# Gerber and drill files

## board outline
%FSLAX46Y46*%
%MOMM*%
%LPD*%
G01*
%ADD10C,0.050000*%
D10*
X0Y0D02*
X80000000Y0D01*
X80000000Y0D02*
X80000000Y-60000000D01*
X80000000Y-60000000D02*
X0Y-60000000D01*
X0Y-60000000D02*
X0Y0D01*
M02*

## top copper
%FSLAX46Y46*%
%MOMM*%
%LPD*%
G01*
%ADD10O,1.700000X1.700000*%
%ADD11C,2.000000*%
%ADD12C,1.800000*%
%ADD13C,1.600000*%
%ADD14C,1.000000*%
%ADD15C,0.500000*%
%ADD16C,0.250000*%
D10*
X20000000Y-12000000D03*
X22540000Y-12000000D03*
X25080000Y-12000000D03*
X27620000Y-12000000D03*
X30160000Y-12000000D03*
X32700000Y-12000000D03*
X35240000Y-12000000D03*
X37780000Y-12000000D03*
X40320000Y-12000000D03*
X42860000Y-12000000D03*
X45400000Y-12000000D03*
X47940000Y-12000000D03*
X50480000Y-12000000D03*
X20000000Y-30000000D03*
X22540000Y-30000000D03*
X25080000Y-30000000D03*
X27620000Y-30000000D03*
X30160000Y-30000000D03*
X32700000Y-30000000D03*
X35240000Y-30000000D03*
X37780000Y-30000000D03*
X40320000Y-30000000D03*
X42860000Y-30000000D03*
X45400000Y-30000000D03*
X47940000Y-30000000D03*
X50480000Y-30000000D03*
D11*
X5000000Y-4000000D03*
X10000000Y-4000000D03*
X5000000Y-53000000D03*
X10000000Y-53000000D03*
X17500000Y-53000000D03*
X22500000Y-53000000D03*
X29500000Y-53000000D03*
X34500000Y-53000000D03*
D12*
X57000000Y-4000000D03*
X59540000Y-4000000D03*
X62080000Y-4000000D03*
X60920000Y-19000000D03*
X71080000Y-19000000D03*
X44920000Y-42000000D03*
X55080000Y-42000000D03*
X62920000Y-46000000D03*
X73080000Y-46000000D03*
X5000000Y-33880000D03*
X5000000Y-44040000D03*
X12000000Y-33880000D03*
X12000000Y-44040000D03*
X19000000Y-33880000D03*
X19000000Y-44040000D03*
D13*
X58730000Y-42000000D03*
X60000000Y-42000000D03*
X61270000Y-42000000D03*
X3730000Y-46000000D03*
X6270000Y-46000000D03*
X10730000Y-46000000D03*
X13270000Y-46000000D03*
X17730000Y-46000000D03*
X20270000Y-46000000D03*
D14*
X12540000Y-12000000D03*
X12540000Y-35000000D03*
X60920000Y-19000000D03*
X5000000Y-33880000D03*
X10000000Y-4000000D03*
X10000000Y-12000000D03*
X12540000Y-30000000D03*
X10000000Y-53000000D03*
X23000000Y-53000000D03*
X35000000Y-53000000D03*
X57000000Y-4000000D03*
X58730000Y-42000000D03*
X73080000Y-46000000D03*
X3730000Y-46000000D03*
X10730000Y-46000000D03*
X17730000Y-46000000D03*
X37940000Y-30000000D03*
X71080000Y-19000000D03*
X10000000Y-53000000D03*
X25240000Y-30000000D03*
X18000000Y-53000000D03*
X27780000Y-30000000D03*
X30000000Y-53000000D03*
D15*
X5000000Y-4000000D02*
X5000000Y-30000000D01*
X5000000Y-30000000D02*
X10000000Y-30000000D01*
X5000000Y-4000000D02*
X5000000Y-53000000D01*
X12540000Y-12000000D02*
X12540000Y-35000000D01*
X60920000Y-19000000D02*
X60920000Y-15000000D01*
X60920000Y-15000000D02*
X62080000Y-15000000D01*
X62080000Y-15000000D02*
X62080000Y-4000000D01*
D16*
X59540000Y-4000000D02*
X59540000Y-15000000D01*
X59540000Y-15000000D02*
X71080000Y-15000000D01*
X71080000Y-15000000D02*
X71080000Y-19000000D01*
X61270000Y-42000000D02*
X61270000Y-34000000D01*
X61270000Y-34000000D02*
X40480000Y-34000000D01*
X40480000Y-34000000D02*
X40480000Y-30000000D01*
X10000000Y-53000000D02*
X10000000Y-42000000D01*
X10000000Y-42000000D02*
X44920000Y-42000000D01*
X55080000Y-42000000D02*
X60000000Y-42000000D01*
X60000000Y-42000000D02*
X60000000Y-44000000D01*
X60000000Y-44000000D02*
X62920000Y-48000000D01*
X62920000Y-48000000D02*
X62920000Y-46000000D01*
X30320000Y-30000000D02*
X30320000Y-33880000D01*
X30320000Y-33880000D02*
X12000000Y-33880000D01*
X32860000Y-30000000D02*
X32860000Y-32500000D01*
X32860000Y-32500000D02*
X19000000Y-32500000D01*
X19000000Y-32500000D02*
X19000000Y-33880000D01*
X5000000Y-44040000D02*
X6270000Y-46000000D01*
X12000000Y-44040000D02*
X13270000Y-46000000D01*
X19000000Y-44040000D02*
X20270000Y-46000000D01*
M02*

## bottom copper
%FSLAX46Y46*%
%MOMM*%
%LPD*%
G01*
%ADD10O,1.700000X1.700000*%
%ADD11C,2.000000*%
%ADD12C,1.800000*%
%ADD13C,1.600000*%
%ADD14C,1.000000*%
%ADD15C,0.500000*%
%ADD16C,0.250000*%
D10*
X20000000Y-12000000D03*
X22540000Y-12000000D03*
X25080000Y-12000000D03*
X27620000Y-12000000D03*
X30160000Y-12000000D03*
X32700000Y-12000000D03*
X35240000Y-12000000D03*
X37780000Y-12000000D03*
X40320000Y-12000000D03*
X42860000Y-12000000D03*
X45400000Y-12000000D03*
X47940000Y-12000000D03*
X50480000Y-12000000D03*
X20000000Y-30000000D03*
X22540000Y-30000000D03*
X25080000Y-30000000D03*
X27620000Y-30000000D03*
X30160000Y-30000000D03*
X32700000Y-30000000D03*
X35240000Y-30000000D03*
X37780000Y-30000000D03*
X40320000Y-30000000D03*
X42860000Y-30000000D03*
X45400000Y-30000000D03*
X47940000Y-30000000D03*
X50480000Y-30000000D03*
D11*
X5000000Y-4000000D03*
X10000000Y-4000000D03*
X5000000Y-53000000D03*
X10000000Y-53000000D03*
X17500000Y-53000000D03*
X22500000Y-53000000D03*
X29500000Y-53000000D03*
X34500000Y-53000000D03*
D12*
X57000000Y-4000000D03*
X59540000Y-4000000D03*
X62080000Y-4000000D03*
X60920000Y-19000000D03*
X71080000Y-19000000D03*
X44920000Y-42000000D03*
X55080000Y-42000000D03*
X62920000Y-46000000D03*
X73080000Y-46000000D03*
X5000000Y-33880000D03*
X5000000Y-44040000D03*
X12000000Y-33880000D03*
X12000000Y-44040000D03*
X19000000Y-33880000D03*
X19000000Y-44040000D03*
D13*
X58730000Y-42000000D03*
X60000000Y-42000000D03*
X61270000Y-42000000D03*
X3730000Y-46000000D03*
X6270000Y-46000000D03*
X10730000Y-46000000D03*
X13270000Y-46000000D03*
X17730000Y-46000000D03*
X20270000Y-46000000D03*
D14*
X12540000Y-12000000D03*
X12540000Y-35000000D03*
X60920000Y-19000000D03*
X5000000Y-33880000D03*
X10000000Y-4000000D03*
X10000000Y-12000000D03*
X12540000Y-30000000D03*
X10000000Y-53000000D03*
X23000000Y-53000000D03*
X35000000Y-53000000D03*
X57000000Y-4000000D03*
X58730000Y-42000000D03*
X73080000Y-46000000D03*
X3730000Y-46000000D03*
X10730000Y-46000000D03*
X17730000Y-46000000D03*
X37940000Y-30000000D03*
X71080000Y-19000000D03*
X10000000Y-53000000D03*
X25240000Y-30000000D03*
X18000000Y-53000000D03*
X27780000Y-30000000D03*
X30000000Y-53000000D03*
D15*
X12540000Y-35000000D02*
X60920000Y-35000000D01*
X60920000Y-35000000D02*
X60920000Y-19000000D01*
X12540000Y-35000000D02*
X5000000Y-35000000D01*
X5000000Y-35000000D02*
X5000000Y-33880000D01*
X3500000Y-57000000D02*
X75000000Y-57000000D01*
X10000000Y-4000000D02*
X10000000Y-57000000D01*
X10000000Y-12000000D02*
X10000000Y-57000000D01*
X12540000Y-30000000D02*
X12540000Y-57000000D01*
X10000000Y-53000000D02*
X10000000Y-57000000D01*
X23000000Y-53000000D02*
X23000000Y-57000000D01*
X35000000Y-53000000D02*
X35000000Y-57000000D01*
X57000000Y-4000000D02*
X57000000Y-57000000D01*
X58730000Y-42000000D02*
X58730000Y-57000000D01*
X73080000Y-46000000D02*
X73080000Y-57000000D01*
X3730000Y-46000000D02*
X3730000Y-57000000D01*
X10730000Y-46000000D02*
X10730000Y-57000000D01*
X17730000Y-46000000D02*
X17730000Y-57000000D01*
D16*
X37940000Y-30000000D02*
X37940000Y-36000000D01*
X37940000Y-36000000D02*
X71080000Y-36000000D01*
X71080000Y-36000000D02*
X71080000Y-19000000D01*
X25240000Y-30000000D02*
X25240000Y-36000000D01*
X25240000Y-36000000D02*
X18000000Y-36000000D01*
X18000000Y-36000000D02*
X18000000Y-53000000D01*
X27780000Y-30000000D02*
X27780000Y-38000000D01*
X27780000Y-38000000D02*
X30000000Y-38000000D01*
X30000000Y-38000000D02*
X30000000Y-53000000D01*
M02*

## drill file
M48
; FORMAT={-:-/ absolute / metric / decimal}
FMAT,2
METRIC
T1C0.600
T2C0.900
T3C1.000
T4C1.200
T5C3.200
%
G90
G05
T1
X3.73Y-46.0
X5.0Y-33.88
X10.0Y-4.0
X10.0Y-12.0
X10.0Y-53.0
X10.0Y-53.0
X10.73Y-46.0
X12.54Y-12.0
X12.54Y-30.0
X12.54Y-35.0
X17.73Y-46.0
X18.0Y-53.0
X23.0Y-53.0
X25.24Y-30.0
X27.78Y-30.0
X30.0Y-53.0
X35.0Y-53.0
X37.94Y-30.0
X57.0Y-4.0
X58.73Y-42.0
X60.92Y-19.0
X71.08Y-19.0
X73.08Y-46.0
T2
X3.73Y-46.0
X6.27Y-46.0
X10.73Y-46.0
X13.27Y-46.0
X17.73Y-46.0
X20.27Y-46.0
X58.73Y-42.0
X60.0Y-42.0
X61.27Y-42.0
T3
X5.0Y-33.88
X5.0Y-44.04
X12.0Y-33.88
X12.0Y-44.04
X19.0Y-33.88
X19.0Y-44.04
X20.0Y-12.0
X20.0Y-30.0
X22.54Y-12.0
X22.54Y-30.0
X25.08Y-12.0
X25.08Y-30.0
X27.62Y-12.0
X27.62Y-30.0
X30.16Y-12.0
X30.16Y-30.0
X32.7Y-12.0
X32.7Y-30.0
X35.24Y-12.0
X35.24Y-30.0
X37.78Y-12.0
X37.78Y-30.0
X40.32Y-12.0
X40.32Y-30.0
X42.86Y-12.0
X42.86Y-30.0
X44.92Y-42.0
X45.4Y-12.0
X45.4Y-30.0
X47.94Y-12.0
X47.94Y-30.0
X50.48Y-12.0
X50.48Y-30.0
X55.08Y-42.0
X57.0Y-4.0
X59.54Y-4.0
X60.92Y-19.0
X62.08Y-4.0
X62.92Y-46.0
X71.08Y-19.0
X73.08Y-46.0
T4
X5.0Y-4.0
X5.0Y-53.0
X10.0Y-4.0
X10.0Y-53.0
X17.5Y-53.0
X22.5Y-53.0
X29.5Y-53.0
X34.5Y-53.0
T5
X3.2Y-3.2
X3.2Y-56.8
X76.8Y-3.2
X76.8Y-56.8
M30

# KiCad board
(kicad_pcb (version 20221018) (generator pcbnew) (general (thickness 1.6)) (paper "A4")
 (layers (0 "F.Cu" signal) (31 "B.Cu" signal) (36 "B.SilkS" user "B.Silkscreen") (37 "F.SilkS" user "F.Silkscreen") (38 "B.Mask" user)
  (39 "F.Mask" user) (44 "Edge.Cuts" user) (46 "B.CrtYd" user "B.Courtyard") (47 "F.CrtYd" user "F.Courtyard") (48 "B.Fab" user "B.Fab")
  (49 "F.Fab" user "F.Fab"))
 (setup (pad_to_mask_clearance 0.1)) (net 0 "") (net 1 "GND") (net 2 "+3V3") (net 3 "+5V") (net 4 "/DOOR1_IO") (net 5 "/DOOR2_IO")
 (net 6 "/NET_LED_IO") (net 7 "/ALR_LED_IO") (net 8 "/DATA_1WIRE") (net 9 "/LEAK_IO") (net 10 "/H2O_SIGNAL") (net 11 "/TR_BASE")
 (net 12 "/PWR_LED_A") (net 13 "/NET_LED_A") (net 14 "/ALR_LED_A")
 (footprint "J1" (layer "F.Cu") (at 25.240 12.000)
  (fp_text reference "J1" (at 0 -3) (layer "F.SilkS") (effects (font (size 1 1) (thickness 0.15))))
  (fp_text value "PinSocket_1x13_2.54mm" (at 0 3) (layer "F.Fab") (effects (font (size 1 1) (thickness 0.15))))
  (pad "1" thru_hole oval (at -5.240 0.000) (size 1.7 1.7) (drill 1.0) (layers "F.Cu" "B.Cu" "F.Mask" "B.Mask") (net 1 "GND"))
  (pad "2" thru_hole oval (at -2.700 0.000) (size 1.7 1.7) (drill 1.0) (layers "F.Cu" "B.Cu" "F.Mask" "B.Mask") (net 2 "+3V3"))
  (pad "3" thru_hole oval (at -0.160 0.000) (size 1.7 1.7) (drill 1.0) (layers "F.Cu" "B.Cu" "F.Mask" "B.Mask"))
  (pad "4" thru_hole oval (at 2.380 0.000) (size 1.7 1.7) (drill 1.0) (layers "F.Cu" "B.Cu" "F.Mask" "B.Mask"))
  (pad "5" thru_hole oval (at 4.920 0.000) (size 1.7 1.7) (drill 1.0) (layers "F.Cu" "B.Cu" "F.Mask" "B.Mask"))
  (pad "6" thru_hole oval (at 7.460 0.000) (size 1.7 1.7) (drill 1.0) (layers "F.Cu" "B.Cu" "F.Mask" "B.Mask"))
  (pad "7" thru_hole oval (at 10.000 0.000) (size 1.7 1.7) (drill 1.0) (layers "F.Cu" "B.Cu" "F.Mask" "B.Mask"))
  (pad "8" thru_hole oval (at 12.540 0.000) (size 1.7 1.7) (drill 1.0) (layers "F.Cu" "B.Cu" "F.Mask" "B.Mask"))
  (pad "9" thru_hole oval (at 15.080 0.000) (size 1.7 1.7) (drill 1.0) (layers "F.Cu" "B.Cu" "F.Mask" "B.Mask"))
  (pad "10" thru_hole oval (at 17.620 0.000) (size 1.7 1.7) (drill 1.0) (layers "F.Cu" "B.Cu" "F.Mask" "B.Mask"))
  (pad "11" thru_hole oval (at 20.160 0.000) (size 1.7 1.7) (drill 1.0) (layers "F.Cu" "B.Cu" "F.Mask" "B.Mask"))
  (pad "12" thru_hole oval (at 22.700 0.000) (size 1.7 1.7) (drill 1.0) (layers "F.Cu" "B.Cu" "F.Mask" "B.Mask"))
  (pad "13" thru_hole oval (at 25.240 0.000) (size 1.7 1.7) (drill 1.0) (layers "F.Cu" "B.Cu" "F.Mask" "B.Mask")))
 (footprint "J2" (layer "F.Cu") (at 25.240 30.000)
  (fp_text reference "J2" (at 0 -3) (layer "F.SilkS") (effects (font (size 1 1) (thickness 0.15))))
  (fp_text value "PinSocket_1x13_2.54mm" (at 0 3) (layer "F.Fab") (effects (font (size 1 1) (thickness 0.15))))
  (pad "1" thru_hole oval (at -5.240 0.000) (size 1.7 1.7) (drill 1.0) (layers "F.Cu" "B.Cu" "F.Mask" "B.Mask") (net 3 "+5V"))
  (pad "2" thru_hole oval (at -2.700 0.000) (size 1.7 1.7) (drill 1.0) (layers "F.Cu" "B.Cu" "F.Mask" "B.Mask") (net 1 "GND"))
  (pad "3" thru_hole oval (at -0.160 0.000) (size 1.7 1.7) (drill 1.0) (layers "F.Cu" "B.Cu" "F.Mask" "B.Mask"))
  (pad "4" thru_hole oval (at 2.380 0.000) (size 1.7 1.7) (drill 1.0) (layers "F.Cu" "B.Cu" "F.Mask" "B.Mask"))
  (pad "5" thru_hole oval (at 4.920 0.000) (size 1.7 1.7) (drill 1.0) (layers "F.Cu" "B.Cu" "F.Mask" "B.Mask"))
  (pad "6" thru_hole oval (at 7.460 0.000) (size 1.7 1.7) (drill 1.0) (layers "F.Cu" "B.Cu" "F.Mask" "B.Mask"))
  (pad "7" thru_hole oval (at 10.000 0.000) (size 1.7 1.7) (drill 1.0) (layers "F.Cu" "B.Cu" "F.Mask" "B.Mask") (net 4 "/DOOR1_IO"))
  (pad "8" thru_hole oval (at 12.540 0.000) (size 1.7 1.7) (drill 1.0) (layers "F.Cu" "B.Cu" "F.Mask" "B.Mask") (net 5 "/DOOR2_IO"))
  (pad "9" thru_hole oval (at 15.080 0.000) (size 1.7 1.7) (drill 1.0) (layers "F.Cu" "B.Cu" "F.Mask" "B.Mask") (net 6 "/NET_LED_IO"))
  (pad "10" thru_hole oval (at 17.620 0.000) (size 1.7 1.7) (drill 1.0) (layers "F.Cu" "B.Cu" "F.Mask" "B.Mask") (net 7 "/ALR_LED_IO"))
  (pad "11" thru_hole oval (at 20.160 0.000) (size 1.7 1.7) (drill 1.0) (layers "F.Cu" "B.Cu" "F.Mask" "B.Mask"))
  (pad "12" thru_hole oval (at 22.700 0.000) (size 1.7 1.7) (drill 1.0) (layers "F.Cu" "B.Cu" "F.Mask" "B.Mask") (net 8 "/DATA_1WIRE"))
  (pad "13" thru_hole oval (at 25.240 0.000) (size 1.7 1.7) (drill 1.0) (layers "F.Cu" "B.Cu" "F.Mask" "B.Mask") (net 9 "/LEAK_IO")))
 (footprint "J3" (layer "F.Cu") (at 7.500 4.000)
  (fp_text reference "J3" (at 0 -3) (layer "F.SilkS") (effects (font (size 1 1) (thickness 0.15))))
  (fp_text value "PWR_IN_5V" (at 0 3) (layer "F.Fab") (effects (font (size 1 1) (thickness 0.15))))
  (pad "1" thru_hole circle (at -2.500 0.000) (size 2.0 2.0) (drill 1.2) (layers "F.Cu" "B.Cu" "F.Mask" "B.Mask") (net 3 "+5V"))
  (pad "2" thru_hole circle (at 2.500 0.000) (size 2.0 2.0) (drill 1.2) (layers "F.Cu" "B.Cu" "F.Mask" "B.Mask") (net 1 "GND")))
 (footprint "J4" (layer "F.Cu") (at 7.500 53.000)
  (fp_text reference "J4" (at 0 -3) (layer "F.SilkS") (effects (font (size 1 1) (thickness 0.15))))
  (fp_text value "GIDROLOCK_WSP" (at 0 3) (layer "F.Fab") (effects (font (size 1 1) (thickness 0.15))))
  (pad "1" thru_hole circle (at -2.500 0.000) (size 2.0 2.0) (drill 1.2) (layers "F.Cu" "B.Cu" "F.Mask" "B.Mask") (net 3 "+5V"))
  (pad "2" thru_hole circle (at 2.500 0.000) (size 2.0 2.0) (drill 1.2) (layers "F.Cu" "B.Cu" "F.Mask" "B.Mask") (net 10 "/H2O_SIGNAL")))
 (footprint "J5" (layer "F.Cu") (at 20.000 53.000)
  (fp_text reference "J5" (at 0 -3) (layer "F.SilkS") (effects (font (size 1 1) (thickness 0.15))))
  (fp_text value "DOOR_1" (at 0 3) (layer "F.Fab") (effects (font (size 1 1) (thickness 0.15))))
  (pad "1" thru_hole circle (at -2.500 0.000) (size 2.0 2.0) (drill 1.2) (layers "F.Cu" "B.Cu" "F.Mask" "B.Mask") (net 4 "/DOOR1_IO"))
  (pad "2" thru_hole circle (at 2.500 0.000) (size 2.0 2.0) (drill 1.2) (layers "F.Cu" "B.Cu" "F.Mask" "B.Mask") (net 1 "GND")))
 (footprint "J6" (layer "F.Cu") (at 32.000 53.000)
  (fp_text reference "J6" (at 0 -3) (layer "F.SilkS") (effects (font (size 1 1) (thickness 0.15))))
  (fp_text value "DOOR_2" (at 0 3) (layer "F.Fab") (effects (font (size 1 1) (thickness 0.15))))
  (pad "1" thru_hole circle (at -2.500 0.000) (size 2.0 2.0) (drill 1.2) (layers "F.Cu" "B.Cu" "F.Mask" "B.Mask") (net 5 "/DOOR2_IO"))
  (pad "2" thru_hole circle (at 2.500 0.000) (size 2.0 2.0) (drill 1.2) (layers "F.Cu" "B.Cu" "F.Mask" "B.Mask") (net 1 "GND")))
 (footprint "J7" (layer "F.Cu") (at 59.540 4.000)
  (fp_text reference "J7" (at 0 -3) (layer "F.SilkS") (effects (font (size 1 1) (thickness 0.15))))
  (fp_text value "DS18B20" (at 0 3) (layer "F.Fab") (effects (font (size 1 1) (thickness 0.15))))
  (pad "1" thru_hole circle (at -2.540 0.000) (size 1.8 1.8) (drill 1.0) (layers "F.Cu" "B.Cu" "F.Mask" "B.Mask") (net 1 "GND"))
  (pad "2" thru_hole circle (at 0.000 0.000) (size 1.8 1.8) (drill 1.0) (layers "F.Cu" "B.Cu" "F.Mask" "B.Mask") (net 8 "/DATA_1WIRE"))
  (pad "3" thru_hole circle (at 2.540 0.000) (size 1.8 1.8) (drill 1.0) (layers "F.Cu" "B.Cu" "F.Mask" "B.Mask") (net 2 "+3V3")))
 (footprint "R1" (layer "F.Cu") (at 66.000 19.000)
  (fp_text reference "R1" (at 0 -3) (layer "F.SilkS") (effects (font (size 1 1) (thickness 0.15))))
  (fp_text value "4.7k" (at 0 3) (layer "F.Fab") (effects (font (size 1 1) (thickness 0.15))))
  (pad "1" thru_hole circle (at -5.080 0.000) (size 1.8 1.8) (drill 1.0) (layers "F.Cu" "B.Cu" "F.Mask" "B.Mask") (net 2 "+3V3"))
  (pad "2" thru_hole circle (at 5.080 0.000) (size 1.8 1.8) (drill 1.0) (layers "F.Cu" "B.Cu" "F.Mask" "B.Mask") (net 8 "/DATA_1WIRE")))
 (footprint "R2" (layer "F.Cu") (at 50.000 42.000)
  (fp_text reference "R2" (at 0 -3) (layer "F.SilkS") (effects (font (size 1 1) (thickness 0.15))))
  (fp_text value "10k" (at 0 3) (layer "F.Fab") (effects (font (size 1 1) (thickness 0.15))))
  (pad "1" thru_hole circle (at -5.080 0.000) (size 1.8 1.8) (drill 1.0) (layers "F.Cu" "B.Cu" "F.Mask" "B.Mask") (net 10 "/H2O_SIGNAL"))
  (pad "2" thru_hole circle (at 5.080 0.000) (size 1.8 1.8) (drill 1.0) (layers "F.Cu" "B.Cu" "F.Mask" "B.Mask") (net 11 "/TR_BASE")))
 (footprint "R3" (layer "F.Cu") (at 68.000 46.000)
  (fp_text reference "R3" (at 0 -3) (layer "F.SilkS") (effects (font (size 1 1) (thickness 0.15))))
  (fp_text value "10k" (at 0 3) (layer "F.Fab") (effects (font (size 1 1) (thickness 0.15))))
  (pad "1" thru_hole circle (at -5.080 0.000) (size 1.8 1.8) (drill 1.0) (layers "F.Cu" "B.Cu" "F.Mask" "B.Mask") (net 11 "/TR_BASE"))
  (pad "2" thru_hole circle (at 5.080 0.000) (size 1.8 1.8) (drill 1.0) (layers "F.Cu" "B.Cu" "F.Mask" "B.Mask") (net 1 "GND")))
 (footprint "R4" (layer "F.Cu") (at 5.000 38.960)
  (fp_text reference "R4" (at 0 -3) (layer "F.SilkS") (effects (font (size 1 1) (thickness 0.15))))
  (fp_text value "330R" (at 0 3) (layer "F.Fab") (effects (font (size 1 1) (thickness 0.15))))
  (pad "1" thru_hole circle (at 0.000 -5.080) (size 1.8 1.8) (drill 1.0) (layers "F.Cu" "B.Cu" "F.Mask" "B.Mask") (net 2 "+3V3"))
  (pad "2" thru_hole circle (at 0.000 5.080) (size 1.8 1.8) (drill 1.0) (layers "F.Cu" "B.Cu" "F.Mask" "B.Mask") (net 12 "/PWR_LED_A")))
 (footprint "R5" (layer "F.Cu") (at 12.000 38.960)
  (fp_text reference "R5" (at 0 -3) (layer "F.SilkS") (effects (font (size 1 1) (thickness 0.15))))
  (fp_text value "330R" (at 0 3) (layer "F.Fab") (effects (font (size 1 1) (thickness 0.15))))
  (pad "1" thru_hole circle (at 0.000 -5.080) (size 1.8 1.8) (drill 1.0) (layers "F.Cu" "B.Cu" "F.Mask" "B.Mask") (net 6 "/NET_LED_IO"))
  (pad "2" thru_hole circle (at 0.000 5.080) (size 1.8 1.8) (drill 1.0) (layers "F.Cu" "B.Cu" "F.Mask" "B.Mask") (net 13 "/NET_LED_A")))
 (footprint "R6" (layer "F.Cu") (at 19.000 38.960)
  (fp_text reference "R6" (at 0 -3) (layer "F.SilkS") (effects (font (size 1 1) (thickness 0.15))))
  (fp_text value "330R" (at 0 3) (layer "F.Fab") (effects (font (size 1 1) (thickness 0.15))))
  (pad "1" thru_hole circle (at 0.000 -5.080) (size 1.8 1.8) (drill 1.0) (layers "F.Cu" "B.Cu" "F.Mask" "B.Mask") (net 7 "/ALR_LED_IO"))
  (pad "2" thru_hole circle (at 0.000 5.080) (size 1.8 1.8) (drill 1.0) (layers "F.Cu" "B.Cu" "F.Mask" "B.Mask") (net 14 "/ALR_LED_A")))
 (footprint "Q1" (layer "F.Cu") (at 60.000 42.000)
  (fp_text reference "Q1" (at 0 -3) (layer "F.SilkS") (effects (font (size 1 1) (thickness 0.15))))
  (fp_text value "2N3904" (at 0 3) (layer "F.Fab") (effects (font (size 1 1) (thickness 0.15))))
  (pad "1" thru_hole circle (at -1.270 0.000) (size 1.6 1.6) (drill 0.9) (layers "F.Cu" "B.Cu" "F.Mask" "B.Mask") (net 1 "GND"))
  (pad "2" thru_hole circle (at 0.000 0.000) (size 1.6 1.6) (drill 0.9) (layers "F.Cu" "B.Cu" "F.Mask" "B.Mask") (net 11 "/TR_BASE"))
  (pad "3" thru_hole circle (at 1.270 0.000) (size 1.6 1.6) (drill 0.9) (layers "F.Cu" "B.Cu" "F.Mask" "B.Mask") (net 9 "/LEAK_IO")))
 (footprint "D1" (layer "F.Cu") (at 5.000 46.000)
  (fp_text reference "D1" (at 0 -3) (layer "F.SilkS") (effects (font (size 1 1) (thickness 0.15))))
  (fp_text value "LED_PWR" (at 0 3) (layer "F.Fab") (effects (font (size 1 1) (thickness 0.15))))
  (pad "K" thru_hole circle (at -1.270 0.000) (size 1.6 1.6) (drill 0.9) (layers "F.Cu" "B.Cu" "F.Mask" "B.Mask") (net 1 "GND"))
  (pad "A" thru_hole circle (at 1.270 0.000) (size 1.6 1.6) (drill 0.9) (layers "F.Cu" "B.Cu" "F.Mask" "B.Mask") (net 12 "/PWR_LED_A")))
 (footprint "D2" (layer "F.Cu") (at 12.000 46.000)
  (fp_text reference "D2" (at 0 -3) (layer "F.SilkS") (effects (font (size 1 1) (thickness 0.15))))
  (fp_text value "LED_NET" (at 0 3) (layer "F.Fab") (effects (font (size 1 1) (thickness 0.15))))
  (pad "K" thru_hole circle (at -1.270 0.000) (size 1.6 1.6) (drill 0.9) (layers "F.Cu" "B.Cu" "F.Mask" "B.Mask") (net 1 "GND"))
  (pad "A" thru_hole circle (at 1.270 0.000) (size 1.6 1.6) (drill 0.9) (layers "F.Cu" "B.Cu" "F.Mask" "B.Mask") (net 13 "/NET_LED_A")))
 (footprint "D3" (layer "F.Cu") (at 19.000 46.000)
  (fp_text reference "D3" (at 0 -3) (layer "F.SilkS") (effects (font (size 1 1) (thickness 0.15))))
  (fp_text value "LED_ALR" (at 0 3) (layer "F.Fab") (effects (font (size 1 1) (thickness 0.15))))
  (pad "K" thru_hole circle (at -1.270 0.000) (size 1.6 1.6) (drill 0.9) (layers "F.Cu" "B.Cu" "F.Mask" "B.Mask") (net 1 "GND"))
  (pad "A" thru_hole circle (at 1.270 0.000) (size 1.6 1.6) (drill 0.9) (layers "F.Cu" "B.Cu" "F.Mask" "B.Mask") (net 14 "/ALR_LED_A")))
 (segment (start 5.000 4.000) (end 5.000 30.000) (width 0.50) (layer "F.Cu") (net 3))
 (segment (start 5.000 30.000) (end 10.000 30.000) (width 0.50) (layer "F.Cu") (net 3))
 (segment (start 5.000 4.000) (end 5.000 53.000) (width 0.50) (layer "F.Cu") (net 3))
 (via (at 12.540 12.000) (size 1.0) (drill 0.6) (layers "F.Cu" "B.Cu") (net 2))
 (segment (start 12.540 12.000) (end 12.540 35.000) (width 0.50) (layer "F.Cu") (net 2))
 (via (at 12.540 35.000) (size 1.0) (drill 0.6) (layers "F.Cu" "B.Cu") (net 2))
 (segment (start 12.540 35.000) (end 60.920 35.000) (width 0.50) (layer "B.Cu") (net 2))
 (segment (start 60.920 35.000) (end 60.920 19.000) (width 0.50) (layer "B.Cu") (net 2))
 (via (at 60.920 19.000) (size 1.0) (drill 0.6) (layers "F.Cu" "B.Cu") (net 2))
 (segment (start 60.920 19.000) (end 60.920 15.000) (width 0.50) (layer "F.Cu") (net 2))
 (segment (start 60.920 15.000) (end 62.080 15.000) (width 0.50) (layer "F.Cu") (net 2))
 (segment (start 62.080 15.000) (end 62.080 4.000) (width 0.50) (layer "F.Cu") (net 2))
 (segment (start 12.540 35.000) (end 5.000 35.000) (width 0.50) (layer "B.Cu") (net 2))
 (segment (start 5.000 35.000) (end 5.000 33.880) (width 0.50) (layer "B.Cu") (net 2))
 (via (at 5.000 33.880) (size 1.0) (drill 0.6) (layers "F.Cu" "B.Cu") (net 2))
 (via (at 10.000 4.000) (size 1.0) (drill 0.6) (layers "F.Cu" "B.Cu") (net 1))
 (via (at 10.000 12.000) (size 1.0) (drill 0.6) (layers "F.Cu" "B.Cu") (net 1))
 (via (at 12.540 30.000) (size 1.0) (drill 0.6) (layers "F.Cu" "B.Cu") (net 1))
 (via (at 10.000 53.000) (size 1.0) (drill 0.6) (layers "F.Cu" "B.Cu") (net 1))
 (via (at 23.000 53.000) (size 1.0) (drill 0.6) (layers "F.Cu" "B.Cu") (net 1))
 (via (at 35.000 53.000) (size 1.0) (drill 0.6) (layers "F.Cu" "B.Cu") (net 1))
 (via (at 57.000 4.000) (size 1.0) (drill 0.6) (layers "F.Cu" "B.Cu") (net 1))
 (via (at 58.730 42.000) (size 1.0) (drill 0.6) (layers "F.Cu" "B.Cu") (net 1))
 (via (at 73.080 46.000) (size 1.0) (drill 0.6) (layers "F.Cu" "B.Cu") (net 1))
 (via (at 3.730 46.000) (size 1.0) (drill 0.6) (layers "F.Cu" "B.Cu") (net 1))
 (via (at 10.730 46.000) (size 1.0) (drill 0.6) (layers "F.Cu" "B.Cu") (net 1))
 (via (at 17.730 46.000) (size 1.0) (drill 0.6) (layers "F.Cu" "B.Cu") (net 1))
 (segment (start 3.500 57.000) (end 75.000 57.000) (width 0.50) (layer "B.Cu") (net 1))
 (segment (start 10.000 4.000) (end 10.000 57.000) (width 0.50) (layer "B.Cu") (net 1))
 (segment (start 10.000 12.000) (end 10.000 57.000) (width 0.50) (layer "B.Cu") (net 1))
 (segment (start 12.540 30.000) (end 12.540 57.000) (width 0.50) (layer "B.Cu") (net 1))
 (segment (start 10.000 53.000) (end 10.000 57.000) (width 0.50) (layer "B.Cu") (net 1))
 (segment (start 23.000 53.000) (end 23.000 57.000) (width 0.50) (layer "B.Cu") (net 1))
 (segment (start 35.000 53.000) (end 35.000 57.000) (width 0.50) (layer "B.Cu") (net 1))
 (segment (start 57.000 4.000) (end 57.000 57.000) (width 0.50) (layer "B.Cu") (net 1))
 (segment (start 58.730 42.000) (end 58.730 57.000) (width 0.50) (layer "B.Cu") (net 1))
 (segment (start 73.080 46.000) (end 73.080 57.000) (width 0.50) (layer "B.Cu") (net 1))
 (segment (start 3.730 46.000) (end 3.730 57.000) (width 0.50) (layer "B.Cu") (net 1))
 (segment (start 10.730 46.000) (end 10.730 57.000) (width 0.50) (layer "B.Cu") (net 1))
 (segment (start 17.730 46.000) (end 17.730 57.000) (width 0.50) (layer "B.Cu") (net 1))
 (via (at 37.940 30.000) (size 1.0) (drill 0.6) (layers "F.Cu" "B.Cu") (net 8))
 (segment (start 37.940 30.000) (end 37.940 36.000) (width 0.25) (layer "B.Cu") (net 8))
 (segment (start 37.940 36.000) (end 71.080 36.000) (width 0.25) (layer "B.Cu") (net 8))
 (segment (start 71.080 36.000) (end 71.080 19.000) (width 0.25) (layer "B.Cu") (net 8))
 (via (at 71.080 19.000) (size 1.0) (drill 0.6) (layers "F.Cu" "B.Cu") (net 8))
 (segment (start 59.540 4.000) (end 59.540 15.000) (width 0.25) (layer "F.Cu") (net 8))
 (segment (start 59.540 15.000) (end 71.080 15.000) (width 0.25) (layer "F.Cu") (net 8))
 (segment (start 71.080 15.000) (end 71.080 19.000) (width 0.25) (layer "F.Cu") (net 8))
 (segment (start 61.270 42.000) (end 61.270 34.000) (width 0.25) (layer "F.Cu") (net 9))
 (segment (start 61.270 34.000) (end 40.480 34.000) (width 0.25) (layer "F.Cu") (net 9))
 (segment (start 40.480 34.000) (end 40.480 30.000) (width 0.25) (layer "F.Cu") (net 9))
 (via (at 10.000 53.000) (size 1.0) (drill 0.6) (layers "F.Cu" "B.Cu") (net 10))
 (segment (start 10.000 53.000) (end 10.000 42.000) (width 0.25) (layer "F.Cu") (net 10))
 (segment (start 10.000 42.000) (end 44.920 42.000) (width 0.25) (layer "F.Cu") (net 10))
 (segment (start 55.080 42.000) (end 60.000 42.000) (width 0.25) (layer "F.Cu") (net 11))
 (segment (start 60.000 42.000) (end 60.000 44.000) (width 0.25) (layer "F.Cu") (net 11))
 (segment (start 60.000 44.000) (end 62.920 48.000) (width 0.25) (layer "F.Cu") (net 11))
 (segment (start 62.920 48.000) (end 62.920 46.000) (width 0.25) (layer "F.Cu") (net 11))
 (via (at 25.240 30.000) (size 1.0) (drill 0.6) (layers "F.Cu" "B.Cu") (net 4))
 (segment (start 25.240 30.000) (end 25.240 36.000) (width 0.25) (layer "B.Cu") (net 4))
 (segment (start 25.240 36.000) (end 18.000 36.000) (width 0.25) (layer "B.Cu") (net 4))
 (segment (start 18.000 36.000) (end 18.000 53.000) (width 0.25) (layer "B.Cu") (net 4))
 (via (at 18.000 53.000) (size 1.0) (drill 0.6) (layers "F.Cu" "B.Cu") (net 4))
 (via (at 27.780 30.000) (size 1.0) (drill 0.6) (layers "F.Cu" "B.Cu") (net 5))
 (segment (start 27.780 30.000) (end 27.780 38.000) (width 0.25) (layer "B.Cu") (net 5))
 (segment (start 27.780 38.000) (end 30.000 38.000) (width 0.25) (layer "B.Cu") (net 5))
 (segment (start 30.000 38.000) (end 30.000 53.000) (width 0.25) (layer "B.Cu") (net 5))
 (via (at 30.000 53.000) (size 1.0) (drill 0.6) (layers "F.Cu" "B.Cu") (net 5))
 (segment (start 30.320 30.000) (end 30.320 33.880) (width 0.25) (layer "F.Cu") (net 6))
 (segment (start 30.320 33.880) (end 12.000 33.880) (width 0.25) (layer "F.Cu") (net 6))
 (segment (start 32.860 30.000) (end 32.860 32.500) (width 0.25) (layer "F.Cu") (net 7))
 (segment (start 32.860 32.500) (end 19.000 32.500) (width 0.25) (layer "F.Cu") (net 7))
 (segment (start 19.000 32.500) (end 19.000 33.880) (width 0.25) (layer "F.Cu") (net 7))
 (segment (start 5.000 44.040) (end 6.270 46.000) (width 0.25) (layer "F.Cu") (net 12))
 (segment (start 12.000 44.040) (end 13.270 46.000) (width 0.25) (layer "F.Cu") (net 13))
 (segment (start 19.000 44.040) (end 20.270 46.000) (width 0.25) (layer "F.Cu") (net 14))
 (gr_line (start 0 0) (end 80.0 0) (layer "Edge.Cuts") (width 0.05))
 (gr_line (start 80.0 0) (end 80.0 60.0) (layer "Edge.Cuts") (width 0.05))
 (gr_line (start 80.0 60.0) (end 0 60.0) (layer "Edge.Cuts") (width 0.05))
 (gr_line (start 0 60.0) (end 0 0) (layer "Edge.Cuts") (width 0.05))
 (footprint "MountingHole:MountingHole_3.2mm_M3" (layer "F.Cu") (at 3.2 3.2)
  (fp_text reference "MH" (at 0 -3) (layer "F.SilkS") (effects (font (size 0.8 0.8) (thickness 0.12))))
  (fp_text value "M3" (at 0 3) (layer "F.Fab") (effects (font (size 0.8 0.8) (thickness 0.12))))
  (pad "" np_thru_hole circle (at 0 0) (size 3.2 3.2) (drill 3.2) (layers "*.Cu" "*.Mask")))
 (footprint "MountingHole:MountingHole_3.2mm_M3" (layer "F.Cu") (at 76.8 3.2)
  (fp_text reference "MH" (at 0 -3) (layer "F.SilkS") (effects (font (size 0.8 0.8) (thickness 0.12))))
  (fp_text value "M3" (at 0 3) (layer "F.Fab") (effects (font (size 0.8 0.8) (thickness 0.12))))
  (pad "" np_thru_hole circle (at 0 0) (size 3.2 3.2) (drill 3.2) (layers "*.Cu" "*.Mask")))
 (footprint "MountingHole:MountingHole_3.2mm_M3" (layer "F.Cu") (at 3.2 56.8)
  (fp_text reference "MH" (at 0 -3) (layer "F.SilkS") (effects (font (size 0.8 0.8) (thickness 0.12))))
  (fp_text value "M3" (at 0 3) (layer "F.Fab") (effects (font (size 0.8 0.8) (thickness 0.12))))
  (pad "" np_thru_hole circle (at 0 0) (size 3.2 3.2) (drill 3.2) (layers "*.Cu" "*.Mask")))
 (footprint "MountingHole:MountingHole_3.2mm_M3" (layer "F.Cu") (at 76.8 56.8)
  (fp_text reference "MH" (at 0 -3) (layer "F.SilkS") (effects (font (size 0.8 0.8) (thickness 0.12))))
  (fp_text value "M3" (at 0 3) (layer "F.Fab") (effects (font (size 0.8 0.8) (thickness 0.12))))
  (pad "" np_thru_hole circle (at 0 0) (size 3.2 3.2) (drill 3.2) (layers "*.Cu" "*.Mask"))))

